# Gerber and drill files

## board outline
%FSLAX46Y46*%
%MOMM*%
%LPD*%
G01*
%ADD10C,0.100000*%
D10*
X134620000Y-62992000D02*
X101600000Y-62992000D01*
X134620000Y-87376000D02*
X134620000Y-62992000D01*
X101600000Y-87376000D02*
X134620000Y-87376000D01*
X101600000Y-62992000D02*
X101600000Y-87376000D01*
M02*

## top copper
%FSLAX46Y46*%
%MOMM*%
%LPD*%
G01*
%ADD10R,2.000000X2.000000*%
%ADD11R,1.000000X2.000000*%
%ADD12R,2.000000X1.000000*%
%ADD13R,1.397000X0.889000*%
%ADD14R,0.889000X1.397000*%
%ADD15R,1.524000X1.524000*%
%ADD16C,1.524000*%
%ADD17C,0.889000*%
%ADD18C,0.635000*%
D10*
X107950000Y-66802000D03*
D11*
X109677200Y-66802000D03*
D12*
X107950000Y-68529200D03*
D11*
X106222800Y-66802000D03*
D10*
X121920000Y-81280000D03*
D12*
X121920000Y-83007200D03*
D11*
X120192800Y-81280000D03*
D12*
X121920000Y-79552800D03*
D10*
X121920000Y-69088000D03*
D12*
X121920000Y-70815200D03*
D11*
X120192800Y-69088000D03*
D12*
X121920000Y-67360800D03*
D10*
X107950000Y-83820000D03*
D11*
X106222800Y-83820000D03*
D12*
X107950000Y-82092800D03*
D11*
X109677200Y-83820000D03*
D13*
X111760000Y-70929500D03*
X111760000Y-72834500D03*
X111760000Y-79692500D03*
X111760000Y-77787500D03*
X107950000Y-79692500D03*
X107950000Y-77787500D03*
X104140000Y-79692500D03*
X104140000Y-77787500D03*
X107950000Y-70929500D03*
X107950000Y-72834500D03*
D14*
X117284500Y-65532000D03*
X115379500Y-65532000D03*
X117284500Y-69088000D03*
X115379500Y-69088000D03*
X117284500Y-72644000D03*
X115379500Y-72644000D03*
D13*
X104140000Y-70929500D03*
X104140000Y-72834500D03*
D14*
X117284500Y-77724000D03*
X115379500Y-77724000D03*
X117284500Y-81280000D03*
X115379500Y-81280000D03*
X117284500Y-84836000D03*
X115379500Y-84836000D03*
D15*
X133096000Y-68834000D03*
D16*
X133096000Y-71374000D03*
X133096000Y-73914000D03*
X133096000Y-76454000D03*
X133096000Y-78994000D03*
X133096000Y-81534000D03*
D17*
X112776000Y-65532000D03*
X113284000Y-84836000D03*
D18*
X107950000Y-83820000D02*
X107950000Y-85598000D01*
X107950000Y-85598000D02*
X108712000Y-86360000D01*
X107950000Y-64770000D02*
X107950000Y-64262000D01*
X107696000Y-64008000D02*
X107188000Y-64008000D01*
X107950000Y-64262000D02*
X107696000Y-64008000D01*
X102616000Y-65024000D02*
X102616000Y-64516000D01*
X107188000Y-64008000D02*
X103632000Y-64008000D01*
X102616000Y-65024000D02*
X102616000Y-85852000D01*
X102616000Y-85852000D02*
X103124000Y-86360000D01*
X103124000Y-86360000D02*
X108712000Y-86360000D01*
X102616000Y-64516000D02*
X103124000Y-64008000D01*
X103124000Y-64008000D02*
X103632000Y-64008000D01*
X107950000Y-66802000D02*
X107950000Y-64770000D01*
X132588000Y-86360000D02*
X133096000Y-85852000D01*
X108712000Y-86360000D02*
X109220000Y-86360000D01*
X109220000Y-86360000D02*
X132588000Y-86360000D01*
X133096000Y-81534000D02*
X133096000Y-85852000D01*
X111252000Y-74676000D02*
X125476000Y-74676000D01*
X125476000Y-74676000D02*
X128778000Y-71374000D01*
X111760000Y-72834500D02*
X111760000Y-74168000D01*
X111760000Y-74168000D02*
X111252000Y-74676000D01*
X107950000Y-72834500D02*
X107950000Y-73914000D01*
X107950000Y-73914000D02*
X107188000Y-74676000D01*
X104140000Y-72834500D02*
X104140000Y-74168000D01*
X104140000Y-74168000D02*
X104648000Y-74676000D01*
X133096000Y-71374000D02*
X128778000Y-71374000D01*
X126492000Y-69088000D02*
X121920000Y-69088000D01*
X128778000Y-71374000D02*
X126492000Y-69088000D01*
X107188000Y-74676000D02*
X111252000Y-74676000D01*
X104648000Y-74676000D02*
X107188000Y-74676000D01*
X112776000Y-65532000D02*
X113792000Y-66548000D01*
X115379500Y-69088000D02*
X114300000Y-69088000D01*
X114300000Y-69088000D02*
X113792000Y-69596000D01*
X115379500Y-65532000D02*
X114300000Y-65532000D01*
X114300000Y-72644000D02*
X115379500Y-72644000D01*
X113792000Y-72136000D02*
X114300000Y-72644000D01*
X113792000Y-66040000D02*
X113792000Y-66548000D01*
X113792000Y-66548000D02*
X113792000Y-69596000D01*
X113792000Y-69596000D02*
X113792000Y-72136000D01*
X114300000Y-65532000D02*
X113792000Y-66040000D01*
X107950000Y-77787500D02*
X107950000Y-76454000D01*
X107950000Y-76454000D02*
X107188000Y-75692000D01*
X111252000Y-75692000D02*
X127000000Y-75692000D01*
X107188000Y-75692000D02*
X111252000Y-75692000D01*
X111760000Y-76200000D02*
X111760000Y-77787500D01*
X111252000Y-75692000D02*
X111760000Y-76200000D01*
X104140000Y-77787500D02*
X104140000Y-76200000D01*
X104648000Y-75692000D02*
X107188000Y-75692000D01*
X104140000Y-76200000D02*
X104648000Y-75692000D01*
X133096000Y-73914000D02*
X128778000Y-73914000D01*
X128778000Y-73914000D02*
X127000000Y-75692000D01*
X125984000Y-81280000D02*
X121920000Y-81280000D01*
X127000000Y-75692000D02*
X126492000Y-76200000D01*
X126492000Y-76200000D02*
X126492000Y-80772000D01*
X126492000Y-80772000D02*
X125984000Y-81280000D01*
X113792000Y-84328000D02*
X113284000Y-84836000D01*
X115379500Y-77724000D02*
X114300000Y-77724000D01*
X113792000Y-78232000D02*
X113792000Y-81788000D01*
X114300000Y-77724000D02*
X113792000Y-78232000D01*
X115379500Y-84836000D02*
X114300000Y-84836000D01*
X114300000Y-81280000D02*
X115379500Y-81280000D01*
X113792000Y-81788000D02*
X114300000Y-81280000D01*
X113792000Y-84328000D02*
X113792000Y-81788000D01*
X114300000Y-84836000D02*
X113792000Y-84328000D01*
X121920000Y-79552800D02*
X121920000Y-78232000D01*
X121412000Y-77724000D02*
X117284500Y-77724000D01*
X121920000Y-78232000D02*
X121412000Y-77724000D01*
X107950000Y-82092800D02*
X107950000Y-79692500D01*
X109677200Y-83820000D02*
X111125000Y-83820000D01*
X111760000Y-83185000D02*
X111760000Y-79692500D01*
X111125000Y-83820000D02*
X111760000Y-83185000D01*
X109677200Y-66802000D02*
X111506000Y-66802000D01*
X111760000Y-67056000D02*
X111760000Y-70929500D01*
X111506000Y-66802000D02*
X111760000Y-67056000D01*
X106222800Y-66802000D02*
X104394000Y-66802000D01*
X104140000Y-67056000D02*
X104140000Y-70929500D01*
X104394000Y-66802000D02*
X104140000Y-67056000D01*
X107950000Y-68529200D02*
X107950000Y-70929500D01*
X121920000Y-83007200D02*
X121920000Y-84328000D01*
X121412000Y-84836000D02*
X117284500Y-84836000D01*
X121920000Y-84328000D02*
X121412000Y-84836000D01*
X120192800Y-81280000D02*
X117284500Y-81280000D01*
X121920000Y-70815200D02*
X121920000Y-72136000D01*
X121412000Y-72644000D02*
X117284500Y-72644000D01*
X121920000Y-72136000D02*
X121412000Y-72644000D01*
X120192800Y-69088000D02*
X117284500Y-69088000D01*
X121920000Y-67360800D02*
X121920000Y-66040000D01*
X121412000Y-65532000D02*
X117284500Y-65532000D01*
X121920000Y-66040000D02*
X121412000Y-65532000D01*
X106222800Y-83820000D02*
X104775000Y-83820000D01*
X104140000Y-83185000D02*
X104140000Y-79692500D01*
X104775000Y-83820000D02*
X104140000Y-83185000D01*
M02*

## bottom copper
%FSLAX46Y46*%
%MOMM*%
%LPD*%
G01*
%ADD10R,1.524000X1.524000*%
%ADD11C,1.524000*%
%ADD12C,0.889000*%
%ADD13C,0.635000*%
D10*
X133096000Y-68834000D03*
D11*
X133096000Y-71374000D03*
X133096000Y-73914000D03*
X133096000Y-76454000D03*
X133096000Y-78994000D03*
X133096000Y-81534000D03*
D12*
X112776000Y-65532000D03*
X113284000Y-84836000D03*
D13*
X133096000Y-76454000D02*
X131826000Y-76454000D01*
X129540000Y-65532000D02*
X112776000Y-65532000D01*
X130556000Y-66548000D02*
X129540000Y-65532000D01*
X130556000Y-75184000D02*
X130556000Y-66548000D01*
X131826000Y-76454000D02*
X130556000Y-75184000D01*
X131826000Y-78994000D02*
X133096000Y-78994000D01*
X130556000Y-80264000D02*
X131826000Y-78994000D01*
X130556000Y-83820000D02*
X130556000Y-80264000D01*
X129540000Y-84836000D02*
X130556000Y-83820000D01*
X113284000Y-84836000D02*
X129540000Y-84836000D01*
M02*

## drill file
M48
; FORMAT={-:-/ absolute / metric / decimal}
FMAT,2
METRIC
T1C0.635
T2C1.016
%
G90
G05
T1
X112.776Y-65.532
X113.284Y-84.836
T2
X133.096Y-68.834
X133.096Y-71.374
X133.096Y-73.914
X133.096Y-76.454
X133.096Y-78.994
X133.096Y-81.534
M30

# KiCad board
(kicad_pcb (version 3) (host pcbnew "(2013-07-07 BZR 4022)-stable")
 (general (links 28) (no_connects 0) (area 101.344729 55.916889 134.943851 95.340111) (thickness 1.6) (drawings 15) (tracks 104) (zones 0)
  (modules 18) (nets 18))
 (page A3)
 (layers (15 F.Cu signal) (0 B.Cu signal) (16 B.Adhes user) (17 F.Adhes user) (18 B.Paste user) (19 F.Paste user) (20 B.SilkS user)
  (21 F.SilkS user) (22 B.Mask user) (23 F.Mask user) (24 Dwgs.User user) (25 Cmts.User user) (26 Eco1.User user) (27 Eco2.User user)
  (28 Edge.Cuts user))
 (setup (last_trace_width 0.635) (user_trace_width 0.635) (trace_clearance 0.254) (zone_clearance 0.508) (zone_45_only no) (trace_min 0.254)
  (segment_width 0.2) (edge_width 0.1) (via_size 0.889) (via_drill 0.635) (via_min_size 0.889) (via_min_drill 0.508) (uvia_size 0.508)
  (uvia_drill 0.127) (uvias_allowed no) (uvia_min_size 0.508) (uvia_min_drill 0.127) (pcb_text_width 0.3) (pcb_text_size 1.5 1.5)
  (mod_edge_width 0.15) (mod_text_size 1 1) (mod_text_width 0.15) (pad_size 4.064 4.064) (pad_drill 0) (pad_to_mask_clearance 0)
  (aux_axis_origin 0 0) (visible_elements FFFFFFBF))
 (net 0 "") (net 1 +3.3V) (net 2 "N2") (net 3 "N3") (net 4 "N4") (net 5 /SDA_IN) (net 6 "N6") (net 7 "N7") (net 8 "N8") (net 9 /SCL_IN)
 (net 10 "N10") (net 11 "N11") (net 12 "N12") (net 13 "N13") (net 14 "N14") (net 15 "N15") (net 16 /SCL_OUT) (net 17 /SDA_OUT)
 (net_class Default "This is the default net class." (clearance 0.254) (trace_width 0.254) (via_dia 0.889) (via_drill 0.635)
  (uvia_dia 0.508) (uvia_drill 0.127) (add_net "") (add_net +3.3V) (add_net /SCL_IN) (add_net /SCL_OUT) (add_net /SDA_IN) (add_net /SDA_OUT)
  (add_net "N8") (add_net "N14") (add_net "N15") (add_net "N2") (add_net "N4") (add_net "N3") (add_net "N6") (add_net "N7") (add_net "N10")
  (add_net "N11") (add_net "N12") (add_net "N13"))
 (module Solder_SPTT (layer F.Cu) (at 107.95 66.802 270)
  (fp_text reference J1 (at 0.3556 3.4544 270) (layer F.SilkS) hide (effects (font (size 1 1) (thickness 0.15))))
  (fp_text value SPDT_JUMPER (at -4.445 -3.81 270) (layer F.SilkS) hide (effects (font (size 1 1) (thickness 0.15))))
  (pad 1 smd rect (at 0 0 270) (size 2 2) (layers F.Cu F.Paste F.Mask) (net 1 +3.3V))
  (pad 2 smd rect (at 0 -1.7272 270) (size 2 1) (layers F.Cu F.Paste F.Mask) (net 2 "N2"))
  (pad 3 smd rect (at 1.7272 0 270) (size 1 2) (layers F.Cu F.Paste F.Mask) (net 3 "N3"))
  (pad 4 smd rect (at 0 1.7272 270) (size 2 1) (layers F.Cu F.Paste F.Mask) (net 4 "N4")))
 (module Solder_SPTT (layer F.Cu) (at 121.92 81.28 180)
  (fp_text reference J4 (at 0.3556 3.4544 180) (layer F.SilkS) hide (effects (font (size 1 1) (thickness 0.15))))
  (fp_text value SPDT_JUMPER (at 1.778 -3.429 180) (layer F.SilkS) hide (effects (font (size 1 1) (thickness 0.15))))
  (pad 1 smd rect (at 0 0 180) (size 2 2) (layers F.Cu F.Paste F.Mask) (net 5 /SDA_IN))
  (pad 2 smd rect (at 0 -1.7272 180) (size 2 1) (layers F.Cu F.Paste F.Mask) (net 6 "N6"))
  (pad 3 smd rect (at 1.7272 0 180) (size 1 2) (layers F.Cu F.Paste F.Mask) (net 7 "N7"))
  (pad 4 smd rect (at 0 1.7272 180) (size 2 1) (layers F.Cu F.Paste F.Mask) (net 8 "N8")))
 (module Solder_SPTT (layer F.Cu) (at 121.92 69.088 180)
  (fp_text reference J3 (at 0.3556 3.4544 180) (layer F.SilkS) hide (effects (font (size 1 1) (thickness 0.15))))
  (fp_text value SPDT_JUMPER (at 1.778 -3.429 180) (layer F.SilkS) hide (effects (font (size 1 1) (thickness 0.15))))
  (pad 1 smd rect (at 0 0 180) (size 2 2) (layers F.Cu F.Paste F.Mask) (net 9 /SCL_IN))
  (pad 2 smd rect (at 0 -1.7272 180) (size 2 1) (layers F.Cu F.Paste F.Mask) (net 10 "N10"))
  (pad 3 smd rect (at 1.7272 0 180) (size 1 2) (layers F.Cu F.Paste F.Mask) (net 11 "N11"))
  (pad 4 smd rect (at 0 1.7272 180) (size 2 1) (layers F.Cu F.Paste F.Mask) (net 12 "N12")))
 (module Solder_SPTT (layer F.Cu) (at 107.95 83.82 90)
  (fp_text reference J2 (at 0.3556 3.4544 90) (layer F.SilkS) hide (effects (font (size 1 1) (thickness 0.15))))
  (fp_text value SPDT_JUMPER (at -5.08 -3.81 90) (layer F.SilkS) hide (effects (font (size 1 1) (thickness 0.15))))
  (pad 1 smd rect (at 0 0 90) (size 2 2) (layers F.Cu F.Paste F.Mask) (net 1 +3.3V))
  (pad 2 smd rect (at 0 -1.7272 90) (size 2 1) (layers F.Cu F.Paste F.Mask) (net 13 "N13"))
  (pad 3 smd rect (at 1.7272 0 90) (size 1 2) (layers F.Cu F.Paste F.Mask) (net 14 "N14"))
  (pad 4 smd rect (at 0 1.7272 90) (size 2 1) (layers F.Cu F.Paste F.Mask) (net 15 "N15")))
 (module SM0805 (layer F.Cu) (at 111.76 71.882 270)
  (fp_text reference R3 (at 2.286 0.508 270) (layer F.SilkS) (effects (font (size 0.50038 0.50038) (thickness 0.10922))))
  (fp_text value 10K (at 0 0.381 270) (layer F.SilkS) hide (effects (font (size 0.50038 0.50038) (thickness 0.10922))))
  (pad 1 smd rect (at -0.9525 0 270) (size 0.889 1.397) (layers F.Cu F.Paste F.Mask) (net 2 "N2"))
  (pad 2 smd rect (at 0.9525 0 270) (size 0.889 1.397) (layers F.Cu F.Paste F.Mask) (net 9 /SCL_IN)))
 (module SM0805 (layer F.Cu) (at 111.76 78.74 90)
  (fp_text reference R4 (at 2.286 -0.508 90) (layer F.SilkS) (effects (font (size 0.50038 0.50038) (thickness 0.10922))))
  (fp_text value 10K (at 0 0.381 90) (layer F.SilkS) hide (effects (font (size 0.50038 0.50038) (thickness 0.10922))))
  (pad 1 smd rect (at -0.9525 0 90) (size 0.889 1.397) (layers F.Cu F.Paste F.Mask) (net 15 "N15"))
  (pad 2 smd rect (at 0.9525 0 90) (size 0.889 1.397) (layers F.Cu F.Paste F.Mask) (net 5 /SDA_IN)))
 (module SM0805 (layer F.Cu) (at 107.95 78.74 90)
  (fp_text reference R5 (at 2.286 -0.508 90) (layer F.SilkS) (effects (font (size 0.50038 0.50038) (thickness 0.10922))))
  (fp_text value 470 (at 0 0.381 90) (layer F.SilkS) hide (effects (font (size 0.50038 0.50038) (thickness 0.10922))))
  (pad 1 smd rect (at -0.9525 0 90) (size 0.889 1.397) (layers F.Cu F.Paste F.Mask) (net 14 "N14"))
  (pad 2 smd rect (at 0.9525 0 90) (size 0.889 1.397) (layers F.Cu F.Paste F.Mask) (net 5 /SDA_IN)))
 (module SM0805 (layer F.Cu) (at 104.14 78.74 90)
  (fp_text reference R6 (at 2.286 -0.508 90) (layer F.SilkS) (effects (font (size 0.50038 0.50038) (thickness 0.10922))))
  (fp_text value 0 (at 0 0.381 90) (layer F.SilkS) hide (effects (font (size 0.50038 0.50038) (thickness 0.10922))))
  (pad 1 smd rect (at -0.9525 0 90) (size 0.889 1.397) (layers F.Cu F.Paste F.Mask) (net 13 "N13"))
  (pad 2 smd rect (at 0.9525 0 90) (size 0.889 1.397) (layers F.Cu F.Paste F.Mask) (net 5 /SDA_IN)))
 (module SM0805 (layer F.Cu) (at 107.95 71.882 270)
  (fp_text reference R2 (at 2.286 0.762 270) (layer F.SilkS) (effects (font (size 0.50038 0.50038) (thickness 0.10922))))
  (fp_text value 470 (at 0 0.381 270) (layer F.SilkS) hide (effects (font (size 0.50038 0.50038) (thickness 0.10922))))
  (pad 1 smd rect (at -0.9525 0 270) (size 0.889 1.397) (layers F.Cu F.Paste F.Mask) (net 3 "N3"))
  (pad 2 smd rect (at 0.9525 0 270) (size 0.889 1.397) (layers F.Cu F.Paste F.Mask) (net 9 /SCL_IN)))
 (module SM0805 (layer F.Cu) (at 116.332 65.532 180)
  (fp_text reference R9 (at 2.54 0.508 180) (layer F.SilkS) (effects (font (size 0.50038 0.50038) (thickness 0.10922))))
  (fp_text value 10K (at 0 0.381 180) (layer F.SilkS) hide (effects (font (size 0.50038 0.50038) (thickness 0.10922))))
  (pad 1 smd rect (at -0.9525 0 180) (size 0.889 1.397) (layers F.Cu F.Paste F.Mask) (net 12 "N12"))
  (pad 2 smd rect (at 0.9525 0 180) (size 0.889 1.397) (layers F.Cu F.Paste F.Mask) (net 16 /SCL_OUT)))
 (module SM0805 (layer F.Cu) (at 116.332 69.088 180)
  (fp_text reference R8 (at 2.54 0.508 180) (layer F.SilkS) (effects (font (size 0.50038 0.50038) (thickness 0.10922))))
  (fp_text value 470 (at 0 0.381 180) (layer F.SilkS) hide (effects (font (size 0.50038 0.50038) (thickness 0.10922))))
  (pad 1 smd rect (at -0.9525 0 180) (size 0.889 1.397) (layers F.Cu F.Paste F.Mask) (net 11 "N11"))
  (pad 2 smd rect (at 0.9525 0 180) (size 0.889 1.397) (layers F.Cu F.Paste F.Mask) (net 16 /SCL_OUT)))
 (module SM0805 (layer F.Cu) (at 116.332 72.644 180)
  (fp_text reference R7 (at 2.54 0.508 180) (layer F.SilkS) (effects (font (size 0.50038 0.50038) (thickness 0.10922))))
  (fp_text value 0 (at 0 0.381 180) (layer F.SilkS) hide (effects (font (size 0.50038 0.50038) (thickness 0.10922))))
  (pad 1 smd rect (at -0.9525 0 180) (size 0.889 1.397) (layers F.Cu F.Paste F.Mask) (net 10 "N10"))
  (pad 2 smd rect (at 0.9525 0 180) (size 0.889 1.397) (layers F.Cu F.Paste F.Mask) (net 16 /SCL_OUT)))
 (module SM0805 (layer F.Cu) (at 104.14 71.882 270)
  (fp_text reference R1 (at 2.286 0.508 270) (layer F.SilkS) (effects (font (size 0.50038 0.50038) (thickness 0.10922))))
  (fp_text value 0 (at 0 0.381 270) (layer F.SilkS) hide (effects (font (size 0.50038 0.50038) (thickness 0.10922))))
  (pad 1 smd rect (at -0.9525 0 270) (size 0.889 1.397) (layers F.Cu F.Paste F.Mask) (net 4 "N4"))
  (pad 2 smd rect (at 0.9525 0 270) (size 0.889 1.397) (layers F.Cu F.Paste F.Mask) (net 9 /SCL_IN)))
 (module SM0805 (layer F.Cu) (at 116.332 77.724 180)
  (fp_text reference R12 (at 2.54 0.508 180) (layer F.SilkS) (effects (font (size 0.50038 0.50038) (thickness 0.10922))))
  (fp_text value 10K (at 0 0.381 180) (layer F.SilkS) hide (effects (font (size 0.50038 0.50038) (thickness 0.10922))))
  (pad 1 smd rect (at -0.9525 0 180) (size 0.889 1.397) (layers F.Cu F.Paste F.Mask) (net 8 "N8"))
  (pad 2 smd rect (at 0.9525 0 180) (size 0.889 1.397) (layers F.Cu F.Paste F.Mask) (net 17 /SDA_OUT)))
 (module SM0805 (layer F.Cu) (at 116.332 81.28 180)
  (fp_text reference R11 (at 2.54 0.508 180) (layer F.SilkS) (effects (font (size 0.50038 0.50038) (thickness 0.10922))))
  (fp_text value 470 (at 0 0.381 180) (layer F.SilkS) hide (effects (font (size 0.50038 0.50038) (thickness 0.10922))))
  (pad 1 smd rect (at -0.9525 0 180) (size 0.889 1.397) (layers F.Cu F.Paste F.Mask) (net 7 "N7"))
  (pad 2 smd rect (at 0.9525 0 180) (size 0.889 1.397) (layers F.Cu F.Paste F.Mask) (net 17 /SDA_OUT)))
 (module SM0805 (layer F.Cu) (at 116.332 84.836 180)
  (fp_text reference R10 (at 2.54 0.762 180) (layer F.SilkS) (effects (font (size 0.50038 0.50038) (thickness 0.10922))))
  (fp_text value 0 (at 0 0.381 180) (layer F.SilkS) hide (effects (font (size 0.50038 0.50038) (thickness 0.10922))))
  (pad 1 smd rect (at -0.9525 0 180) (size 0.889 1.397) (layers F.Cu F.Paste F.Mask) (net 6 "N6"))
  (pad 2 smd rect (at 0.9525 0 180) (size 0.889 1.397) (layers F.Cu F.Paste F.Mask) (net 17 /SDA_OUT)))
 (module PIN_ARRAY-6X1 (layer F.Cu) (at 133.096 75.184 270)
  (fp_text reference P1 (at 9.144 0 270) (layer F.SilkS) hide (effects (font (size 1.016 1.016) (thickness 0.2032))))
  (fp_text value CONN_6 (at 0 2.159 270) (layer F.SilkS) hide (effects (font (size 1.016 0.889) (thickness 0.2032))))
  (pad 1 thru_hole rect (at -6.35 0 270) (size 1.524 1.524) (drill 1.016) (layers *.Cu *.Mask F.SilkS))
  (pad 2 thru_hole circle (at -3.81 0 270) (size 1.524 1.524) (drill 1.016) (layers *.Cu *.Mask F.SilkS) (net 9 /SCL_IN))
  (pad 3 thru_hole circle (at -1.27 0 270) (size 1.524 1.524) (drill 1.016) (layers *.Cu *.Mask F.SilkS) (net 5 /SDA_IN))
  (pad 4 thru_hole circle (at 1.27 0 270) (size 1.524 1.524) (drill 1.016) (layers *.Cu *.Mask F.SilkS) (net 16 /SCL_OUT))
  (pad 5 thru_hole circle (at 3.81 0 270) (size 1.524 1.524) (drill 1.016) (layers *.Cu *.Mask F.SilkS) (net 17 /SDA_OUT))
  (pad 6 thru_hole circle (at 6.35 0 270) (size 1.524 1.524) (drill 1.016) (layers *.Cu *.Mask F.SilkS) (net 1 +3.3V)))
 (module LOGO (layer B.Cu) (at 118.364 75.184 180)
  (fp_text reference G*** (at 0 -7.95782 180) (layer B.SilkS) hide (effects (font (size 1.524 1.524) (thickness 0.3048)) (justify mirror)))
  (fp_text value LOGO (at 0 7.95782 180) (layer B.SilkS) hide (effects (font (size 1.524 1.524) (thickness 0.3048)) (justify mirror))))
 (gr_line (start 134.62 62.992) (end 101.6 62.992) (angle 90) (layer Edge.Cuts) (width 0.1))
 (gr_line (start 134.62 87.376) (end 134.62 62.992) (angle 90) (layer Edge.Cuts) (width 0.1))
 (gr_line (start 101.6 87.376) (end 134.62 87.376) (angle 90) (layer Edge.Cuts) (width 0.1))
 (gr_line (start 101.6 62.992) (end 101.6 87.376) (angle 90) (layer Edge.Cuts) (width 0.1))
 (segment (start 107.95 83.82) (end 107.95 85.598) (width 0.635) (layer F.Cu) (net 1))
 (segment (start 107.95 85.598) (end 108.712 86.36) (width 0.635) (layer F.Cu) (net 1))
 (segment (start 107.95 64.77) (end 107.95 64.262) (width 0.635) (layer F.Cu) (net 1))
 (segment (start 107.696 64.008) (end 107.188 64.008) (width 0.635) (layer F.Cu) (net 1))
 (segment (start 107.95 64.262) (end 107.696 64.008) (width 0.635) (layer F.Cu) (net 1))
 (segment (start 102.616 65.024) (end 102.616 64.516) (width 0.635) (layer F.Cu) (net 1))
 (segment (start 107.188 64.008) (end 103.632 64.008) (width 0.635) (layer F.Cu) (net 1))
 (segment (start 102.616 65.024) (end 102.616 85.852) (width 0.635) (layer F.Cu) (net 1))
 (segment (start 102.616 85.852) (end 103.124 86.36) (width 0.635) (layer F.Cu) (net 1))
 (segment (start 103.124 86.36) (end 108.712 86.36) (width 0.635) (layer F.Cu) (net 1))
 (segment (start 102.616 64.516) (end 103.124 64.008) (width 0.635) (layer F.Cu) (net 1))
 (segment (start 103.124 64.008) (end 103.632 64.008) (width 0.635) (layer F.Cu) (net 1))
 (segment (start 107.95 66.802) (end 107.95 64.77) (width 0.635) (layer F.Cu) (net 1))
 (segment (start 132.588 86.36) (end 133.096 85.852) (width 0.635) (layer F.Cu) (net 1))
 (segment (start 108.712 86.36) (end 109.22 86.36) (width 0.635) (layer F.Cu) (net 1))
 (segment (start 109.22 86.36) (end 132.588 86.36) (width 0.635) (layer F.Cu) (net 1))
 (segment (start 133.096 81.534) (end 133.096 85.852) (width 0.635) (layer F.Cu) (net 1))
 (segment (start 111.252 74.676) (end 125.476 74.676) (width 0.635) (layer F.Cu) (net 9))
 (segment (start 125.476 74.676) (end 128.778 71.374) (width 0.635) (layer F.Cu) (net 9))
 (segment (start 111.76 72.8345) (end 111.76 74.168) (width 0.635) (layer F.Cu) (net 9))
 (segment (start 111.76 74.168) (end 111.252 74.676) (width 0.635) (layer F.Cu) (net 9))
 (segment (start 107.95 72.8345) (end 107.95 73.914) (width 0.635) (layer F.Cu) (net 9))
 (segment (start 107.95 73.914) (end 107.188 74.676) (width 0.635) (layer F.Cu) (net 9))
 (segment (start 104.14 72.8345) (end 104.14 74.168) (width 0.635) (layer F.Cu) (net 9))
 (segment (start 104.14 74.168) (end 104.648 74.676) (width 0.635) (layer F.Cu) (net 9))
 (segment (start 133.096 71.374) (end 128.778 71.374) (width 0.635) (layer F.Cu) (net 9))
 (segment (start 126.492 69.088) (end 121.92 69.088) (width 0.635) (layer F.Cu) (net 9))
 (segment (start 128.778 71.374) (end 126.492 69.088) (width 0.635) (layer F.Cu) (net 9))
 (segment (start 107.188 74.676) (end 111.252 74.676) (width 0.635) (layer F.Cu) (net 9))
 (segment (start 104.648 74.676) (end 107.188 74.676) (width 0.635) (layer F.Cu) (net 9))
 (segment (start 133.096 76.454) (end 131.826 76.454) (width 0.635) (layer B.Cu) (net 16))
 (segment (start 112.776 65.532) (end 113.792 66.548) (width 0.635) (layer F.Cu) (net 16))
 (via (at 112.776 65.532) (size 0.889) (layers F.Cu B.Cu) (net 16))
 (segment (start 129.54 65.532) (end 112.776 65.532) (width 0.635) (layer B.Cu) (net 16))
 (segment (start 130.556 66.548) (end 129.54 65.532) (width 0.635) (layer B.Cu) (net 16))
 (segment (start 130.556 75.184) (end 130.556 66.548) (width 0.635) (layer B.Cu) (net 16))
 (segment (start 131.826 76.454) (end 130.556 75.184) (width 0.635) (layer B.Cu) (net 16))
 (segment (start 115.3795 69.088) (end 114.3 69.088) (width 0.635) (layer F.Cu) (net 16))
 (segment (start 114.3 69.088) (end 113.792 69.596) (width 0.635) (layer F.Cu) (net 16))
 (segment (start 115.3795 65.532) (end 114.3 65.532) (width 0.635) (layer F.Cu) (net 16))
 (segment (start 114.3 72.644) (end 115.3795 72.644) (width 0.635) (layer F.Cu) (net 16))
 (segment (start 113.792 72.136) (end 114.3 72.644) (width 0.635) (layer F.Cu) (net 16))
 (segment (start 113.792 66.04) (end 113.792 66.548) (width 0.635) (layer F.Cu) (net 16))
 (segment (start 113.792 66.548) (end 113.792 69.596) (width 0.635) (layer F.Cu) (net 16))
 (segment (start 113.792 69.596) (end 113.792 72.136) (width 0.635) (layer F.Cu) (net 16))
 (segment (start 114.3 65.532) (end 113.792 66.04) (width 0.635) (layer F.Cu) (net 16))
 (segment (start 107.95 77.7875) (end 107.95 76.454) (width 0.635) (layer F.Cu) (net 5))
 (segment (start 107.95 76.454) (end 107.188 75.692) (width 0.635) (layer F.Cu) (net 5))
 (segment (start 111.252 75.692) (end 127 75.692) (width 0.635) (layer F.Cu) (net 5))
 (segment (start 107.188 75.692) (end 111.252 75.692) (width 0.635) (layer F.Cu) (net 5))
 (segment (start 111.76 76.2) (end 111.76 77.7875) (width 0.635) (layer F.Cu) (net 5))
 (segment (start 111.252 75.692) (end 111.76 76.2) (width 0.635) (layer F.Cu) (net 5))
 (segment (start 104.14 77.7875) (end 104.14 76.2) (width 0.635) (layer F.Cu) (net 5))
 (segment (start 104.648 75.692) (end 107.188 75.692) (width 0.635) (layer F.Cu) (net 5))
 (segment (start 104.14 76.2) (end 104.648 75.692) (width 0.635) (layer F.Cu) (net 5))
 (segment (start 133.096 73.914) (end 128.778 73.914) (width 0.635) (layer F.Cu) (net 5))
 (segment (start 128.778 73.914) (end 127 75.692) (width 0.635) (layer F.Cu) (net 5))
 (segment (start 125.984 81.28) (end 121.92 81.28) (width 0.635) (layer F.Cu) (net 5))
 (segment (start 127 75.692) (end 126.492 76.2) (width 0.635) (layer F.Cu) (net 5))
 (segment (start 126.492 76.2) (end 126.492 80.772) (width 0.635) (layer F.Cu) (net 5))
 (segment (start 126.492 80.772) (end 125.984 81.28) (width 0.635) (layer F.Cu) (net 5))
 (segment (start 113.792 84.328) (end 113.284 84.836) (width 0.635) (layer F.Cu) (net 17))
 (segment (start 131.826 78.994) (end 133.096 78.994) (width 0.635) (layer B.Cu) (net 17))
 (segment (start 130.556 80.264) (end 131.826 78.994) (width 0.635) (layer B.Cu) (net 17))
 (segment (start 130.556 83.82) (end 130.556 80.264) (width 0.635) (layer B.Cu) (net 17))
 (segment (start 129.54 84.836) (end 130.556 83.82) (width 0.635) (layer B.Cu) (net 17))
 (segment (start 113.284 84.836) (end 129.54 84.836) (width 0.635) (layer B.Cu) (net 17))
 (via (at 113.284 84.836) (size 0.889) (layers F.Cu B.Cu) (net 17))
 (segment (start 115.3795 77.724) (end 114.3 77.724) (width 0.635) (layer F.Cu) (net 17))
 (segment (start 113.792 78.232) (end 113.792 81.788) (width 0.635) (layer F.Cu) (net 17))
 (segment (start 114.3 77.724) (end 113.792 78.232) (width 0.635) (layer F.Cu) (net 17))
 (segment (start 115.3795 84.836) (end 114.3 84.836) (width 0.635) (layer F.Cu) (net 17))
 (segment (start 114.3 81.28) (end 115.3795 81.28) (width 0.635) (layer F.Cu) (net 17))
 (segment (start 113.792 81.788) (end 114.3 81.28) (width 0.635) (layer F.Cu) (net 17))
 (segment (start 113.792 84.328) (end 113.792 81.788) (width 0.635) (layer F.Cu) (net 17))
 (segment (start 114.3 84.836) (end 113.792 84.328) (width 0.635) (layer F.Cu) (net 17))
 (segment (start 121.92 79.5528) (end 121.92 78.232) (width 0.635) (layer F.Cu) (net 8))
 (segment (start 121.412 77.724) (end 117.2845 77.724) (width 0.635) (layer F.Cu) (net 8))
 (segment (start 121.92 78.232) (end 121.412 77.724) (width 0.635) (layer F.Cu) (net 8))
 (segment (start 107.95 82.0928) (end 107.95 79.6925) (width 0.635) (layer F.Cu) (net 14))
 (segment (start 109.6772 83.82) (end 111.125 83.82) (width 0.635) (layer F.Cu) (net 15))
 (segment (start 111.76 83.185) (end 111.76 79.6925) (width 0.635) (layer F.Cu) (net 15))
 (segment (start 111.125 83.82) (end 111.76 83.185) (width 0.635) (layer F.Cu) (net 15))
 (segment (start 109.6772 66.802) (end 111.506 66.802) (width 0.635) (layer F.Cu) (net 2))
 (segment (start 111.76 67.056) (end 111.76 70.9295) (width 0.635) (layer F.Cu) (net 2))
 (segment (start 111.506 66.802) (end 111.76 67.056) (width 0.635) (layer F.Cu) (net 2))
 (segment (start 106.2228 66.802) (end 104.394 66.802) (width 0.635) (layer F.Cu) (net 4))
 (segment (start 104.14 67.056) (end 104.14 70.9295) (width 0.635) (layer F.Cu) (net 4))
 (segment (start 104.394 66.802) (end 104.14 67.056) (width 0.635) (layer F.Cu) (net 4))
 (segment (start 107.95 68.5292) (end 107.95 70.9295) (width 0.635) (layer F.Cu) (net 3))
 (segment (start 121.92 83.0072) (end 121.92 84.328) (width 0.635) (layer F.Cu) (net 6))
 (segment (start 121.412 84.836) (end 117.2845 84.836) (width 0.635) (layer F.Cu) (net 6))
 (segment (start 121.92 84.328) (end 121.412 84.836) (width 0.635) (layer F.Cu) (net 6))
 (segment (start 120.1928 81.28) (end 117.2845 81.28) (width 0.635) (layer F.Cu) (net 7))
 (segment (start 121.92 70.8152) (end 121.92 72.136) (width 0.635) (layer F.Cu) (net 10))
 (segment (start 121.412 72.644) (end 117.2845 72.644) (width 0.635) (layer F.Cu) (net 10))
 (segment (start 121.92 72.136) (end 121.412 72.644) (width 0.635) (layer F.Cu) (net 10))
 (segment (start 120.1928 69.088) (end 117.2845 69.088) (width 0.635) (layer F.Cu) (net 11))
 (segment (start 121.92 67.3608) (end 121.92 66.04) (width 0.635) (layer F.Cu) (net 12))
 (segment (start 121.412 65.532) (end 117.2845 65.532) (width 0.635) (layer F.Cu) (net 12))
 (segment (start 121.92 66.04) (end 121.412 65.532) (width 0.635) (layer F.Cu) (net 12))
 (segment (start 106.2228 83.82) (end 104.775 83.82) (width 0.635) (layer F.Cu) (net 13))
 (segment (start 104.14 83.185) (end 104.14 79.6925) (width 0.635) (layer F.Cu) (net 13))
 (segment (start 104.775 83.82) (end 104.14 83.185) (width 0.635) (layer F.Cu) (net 13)))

